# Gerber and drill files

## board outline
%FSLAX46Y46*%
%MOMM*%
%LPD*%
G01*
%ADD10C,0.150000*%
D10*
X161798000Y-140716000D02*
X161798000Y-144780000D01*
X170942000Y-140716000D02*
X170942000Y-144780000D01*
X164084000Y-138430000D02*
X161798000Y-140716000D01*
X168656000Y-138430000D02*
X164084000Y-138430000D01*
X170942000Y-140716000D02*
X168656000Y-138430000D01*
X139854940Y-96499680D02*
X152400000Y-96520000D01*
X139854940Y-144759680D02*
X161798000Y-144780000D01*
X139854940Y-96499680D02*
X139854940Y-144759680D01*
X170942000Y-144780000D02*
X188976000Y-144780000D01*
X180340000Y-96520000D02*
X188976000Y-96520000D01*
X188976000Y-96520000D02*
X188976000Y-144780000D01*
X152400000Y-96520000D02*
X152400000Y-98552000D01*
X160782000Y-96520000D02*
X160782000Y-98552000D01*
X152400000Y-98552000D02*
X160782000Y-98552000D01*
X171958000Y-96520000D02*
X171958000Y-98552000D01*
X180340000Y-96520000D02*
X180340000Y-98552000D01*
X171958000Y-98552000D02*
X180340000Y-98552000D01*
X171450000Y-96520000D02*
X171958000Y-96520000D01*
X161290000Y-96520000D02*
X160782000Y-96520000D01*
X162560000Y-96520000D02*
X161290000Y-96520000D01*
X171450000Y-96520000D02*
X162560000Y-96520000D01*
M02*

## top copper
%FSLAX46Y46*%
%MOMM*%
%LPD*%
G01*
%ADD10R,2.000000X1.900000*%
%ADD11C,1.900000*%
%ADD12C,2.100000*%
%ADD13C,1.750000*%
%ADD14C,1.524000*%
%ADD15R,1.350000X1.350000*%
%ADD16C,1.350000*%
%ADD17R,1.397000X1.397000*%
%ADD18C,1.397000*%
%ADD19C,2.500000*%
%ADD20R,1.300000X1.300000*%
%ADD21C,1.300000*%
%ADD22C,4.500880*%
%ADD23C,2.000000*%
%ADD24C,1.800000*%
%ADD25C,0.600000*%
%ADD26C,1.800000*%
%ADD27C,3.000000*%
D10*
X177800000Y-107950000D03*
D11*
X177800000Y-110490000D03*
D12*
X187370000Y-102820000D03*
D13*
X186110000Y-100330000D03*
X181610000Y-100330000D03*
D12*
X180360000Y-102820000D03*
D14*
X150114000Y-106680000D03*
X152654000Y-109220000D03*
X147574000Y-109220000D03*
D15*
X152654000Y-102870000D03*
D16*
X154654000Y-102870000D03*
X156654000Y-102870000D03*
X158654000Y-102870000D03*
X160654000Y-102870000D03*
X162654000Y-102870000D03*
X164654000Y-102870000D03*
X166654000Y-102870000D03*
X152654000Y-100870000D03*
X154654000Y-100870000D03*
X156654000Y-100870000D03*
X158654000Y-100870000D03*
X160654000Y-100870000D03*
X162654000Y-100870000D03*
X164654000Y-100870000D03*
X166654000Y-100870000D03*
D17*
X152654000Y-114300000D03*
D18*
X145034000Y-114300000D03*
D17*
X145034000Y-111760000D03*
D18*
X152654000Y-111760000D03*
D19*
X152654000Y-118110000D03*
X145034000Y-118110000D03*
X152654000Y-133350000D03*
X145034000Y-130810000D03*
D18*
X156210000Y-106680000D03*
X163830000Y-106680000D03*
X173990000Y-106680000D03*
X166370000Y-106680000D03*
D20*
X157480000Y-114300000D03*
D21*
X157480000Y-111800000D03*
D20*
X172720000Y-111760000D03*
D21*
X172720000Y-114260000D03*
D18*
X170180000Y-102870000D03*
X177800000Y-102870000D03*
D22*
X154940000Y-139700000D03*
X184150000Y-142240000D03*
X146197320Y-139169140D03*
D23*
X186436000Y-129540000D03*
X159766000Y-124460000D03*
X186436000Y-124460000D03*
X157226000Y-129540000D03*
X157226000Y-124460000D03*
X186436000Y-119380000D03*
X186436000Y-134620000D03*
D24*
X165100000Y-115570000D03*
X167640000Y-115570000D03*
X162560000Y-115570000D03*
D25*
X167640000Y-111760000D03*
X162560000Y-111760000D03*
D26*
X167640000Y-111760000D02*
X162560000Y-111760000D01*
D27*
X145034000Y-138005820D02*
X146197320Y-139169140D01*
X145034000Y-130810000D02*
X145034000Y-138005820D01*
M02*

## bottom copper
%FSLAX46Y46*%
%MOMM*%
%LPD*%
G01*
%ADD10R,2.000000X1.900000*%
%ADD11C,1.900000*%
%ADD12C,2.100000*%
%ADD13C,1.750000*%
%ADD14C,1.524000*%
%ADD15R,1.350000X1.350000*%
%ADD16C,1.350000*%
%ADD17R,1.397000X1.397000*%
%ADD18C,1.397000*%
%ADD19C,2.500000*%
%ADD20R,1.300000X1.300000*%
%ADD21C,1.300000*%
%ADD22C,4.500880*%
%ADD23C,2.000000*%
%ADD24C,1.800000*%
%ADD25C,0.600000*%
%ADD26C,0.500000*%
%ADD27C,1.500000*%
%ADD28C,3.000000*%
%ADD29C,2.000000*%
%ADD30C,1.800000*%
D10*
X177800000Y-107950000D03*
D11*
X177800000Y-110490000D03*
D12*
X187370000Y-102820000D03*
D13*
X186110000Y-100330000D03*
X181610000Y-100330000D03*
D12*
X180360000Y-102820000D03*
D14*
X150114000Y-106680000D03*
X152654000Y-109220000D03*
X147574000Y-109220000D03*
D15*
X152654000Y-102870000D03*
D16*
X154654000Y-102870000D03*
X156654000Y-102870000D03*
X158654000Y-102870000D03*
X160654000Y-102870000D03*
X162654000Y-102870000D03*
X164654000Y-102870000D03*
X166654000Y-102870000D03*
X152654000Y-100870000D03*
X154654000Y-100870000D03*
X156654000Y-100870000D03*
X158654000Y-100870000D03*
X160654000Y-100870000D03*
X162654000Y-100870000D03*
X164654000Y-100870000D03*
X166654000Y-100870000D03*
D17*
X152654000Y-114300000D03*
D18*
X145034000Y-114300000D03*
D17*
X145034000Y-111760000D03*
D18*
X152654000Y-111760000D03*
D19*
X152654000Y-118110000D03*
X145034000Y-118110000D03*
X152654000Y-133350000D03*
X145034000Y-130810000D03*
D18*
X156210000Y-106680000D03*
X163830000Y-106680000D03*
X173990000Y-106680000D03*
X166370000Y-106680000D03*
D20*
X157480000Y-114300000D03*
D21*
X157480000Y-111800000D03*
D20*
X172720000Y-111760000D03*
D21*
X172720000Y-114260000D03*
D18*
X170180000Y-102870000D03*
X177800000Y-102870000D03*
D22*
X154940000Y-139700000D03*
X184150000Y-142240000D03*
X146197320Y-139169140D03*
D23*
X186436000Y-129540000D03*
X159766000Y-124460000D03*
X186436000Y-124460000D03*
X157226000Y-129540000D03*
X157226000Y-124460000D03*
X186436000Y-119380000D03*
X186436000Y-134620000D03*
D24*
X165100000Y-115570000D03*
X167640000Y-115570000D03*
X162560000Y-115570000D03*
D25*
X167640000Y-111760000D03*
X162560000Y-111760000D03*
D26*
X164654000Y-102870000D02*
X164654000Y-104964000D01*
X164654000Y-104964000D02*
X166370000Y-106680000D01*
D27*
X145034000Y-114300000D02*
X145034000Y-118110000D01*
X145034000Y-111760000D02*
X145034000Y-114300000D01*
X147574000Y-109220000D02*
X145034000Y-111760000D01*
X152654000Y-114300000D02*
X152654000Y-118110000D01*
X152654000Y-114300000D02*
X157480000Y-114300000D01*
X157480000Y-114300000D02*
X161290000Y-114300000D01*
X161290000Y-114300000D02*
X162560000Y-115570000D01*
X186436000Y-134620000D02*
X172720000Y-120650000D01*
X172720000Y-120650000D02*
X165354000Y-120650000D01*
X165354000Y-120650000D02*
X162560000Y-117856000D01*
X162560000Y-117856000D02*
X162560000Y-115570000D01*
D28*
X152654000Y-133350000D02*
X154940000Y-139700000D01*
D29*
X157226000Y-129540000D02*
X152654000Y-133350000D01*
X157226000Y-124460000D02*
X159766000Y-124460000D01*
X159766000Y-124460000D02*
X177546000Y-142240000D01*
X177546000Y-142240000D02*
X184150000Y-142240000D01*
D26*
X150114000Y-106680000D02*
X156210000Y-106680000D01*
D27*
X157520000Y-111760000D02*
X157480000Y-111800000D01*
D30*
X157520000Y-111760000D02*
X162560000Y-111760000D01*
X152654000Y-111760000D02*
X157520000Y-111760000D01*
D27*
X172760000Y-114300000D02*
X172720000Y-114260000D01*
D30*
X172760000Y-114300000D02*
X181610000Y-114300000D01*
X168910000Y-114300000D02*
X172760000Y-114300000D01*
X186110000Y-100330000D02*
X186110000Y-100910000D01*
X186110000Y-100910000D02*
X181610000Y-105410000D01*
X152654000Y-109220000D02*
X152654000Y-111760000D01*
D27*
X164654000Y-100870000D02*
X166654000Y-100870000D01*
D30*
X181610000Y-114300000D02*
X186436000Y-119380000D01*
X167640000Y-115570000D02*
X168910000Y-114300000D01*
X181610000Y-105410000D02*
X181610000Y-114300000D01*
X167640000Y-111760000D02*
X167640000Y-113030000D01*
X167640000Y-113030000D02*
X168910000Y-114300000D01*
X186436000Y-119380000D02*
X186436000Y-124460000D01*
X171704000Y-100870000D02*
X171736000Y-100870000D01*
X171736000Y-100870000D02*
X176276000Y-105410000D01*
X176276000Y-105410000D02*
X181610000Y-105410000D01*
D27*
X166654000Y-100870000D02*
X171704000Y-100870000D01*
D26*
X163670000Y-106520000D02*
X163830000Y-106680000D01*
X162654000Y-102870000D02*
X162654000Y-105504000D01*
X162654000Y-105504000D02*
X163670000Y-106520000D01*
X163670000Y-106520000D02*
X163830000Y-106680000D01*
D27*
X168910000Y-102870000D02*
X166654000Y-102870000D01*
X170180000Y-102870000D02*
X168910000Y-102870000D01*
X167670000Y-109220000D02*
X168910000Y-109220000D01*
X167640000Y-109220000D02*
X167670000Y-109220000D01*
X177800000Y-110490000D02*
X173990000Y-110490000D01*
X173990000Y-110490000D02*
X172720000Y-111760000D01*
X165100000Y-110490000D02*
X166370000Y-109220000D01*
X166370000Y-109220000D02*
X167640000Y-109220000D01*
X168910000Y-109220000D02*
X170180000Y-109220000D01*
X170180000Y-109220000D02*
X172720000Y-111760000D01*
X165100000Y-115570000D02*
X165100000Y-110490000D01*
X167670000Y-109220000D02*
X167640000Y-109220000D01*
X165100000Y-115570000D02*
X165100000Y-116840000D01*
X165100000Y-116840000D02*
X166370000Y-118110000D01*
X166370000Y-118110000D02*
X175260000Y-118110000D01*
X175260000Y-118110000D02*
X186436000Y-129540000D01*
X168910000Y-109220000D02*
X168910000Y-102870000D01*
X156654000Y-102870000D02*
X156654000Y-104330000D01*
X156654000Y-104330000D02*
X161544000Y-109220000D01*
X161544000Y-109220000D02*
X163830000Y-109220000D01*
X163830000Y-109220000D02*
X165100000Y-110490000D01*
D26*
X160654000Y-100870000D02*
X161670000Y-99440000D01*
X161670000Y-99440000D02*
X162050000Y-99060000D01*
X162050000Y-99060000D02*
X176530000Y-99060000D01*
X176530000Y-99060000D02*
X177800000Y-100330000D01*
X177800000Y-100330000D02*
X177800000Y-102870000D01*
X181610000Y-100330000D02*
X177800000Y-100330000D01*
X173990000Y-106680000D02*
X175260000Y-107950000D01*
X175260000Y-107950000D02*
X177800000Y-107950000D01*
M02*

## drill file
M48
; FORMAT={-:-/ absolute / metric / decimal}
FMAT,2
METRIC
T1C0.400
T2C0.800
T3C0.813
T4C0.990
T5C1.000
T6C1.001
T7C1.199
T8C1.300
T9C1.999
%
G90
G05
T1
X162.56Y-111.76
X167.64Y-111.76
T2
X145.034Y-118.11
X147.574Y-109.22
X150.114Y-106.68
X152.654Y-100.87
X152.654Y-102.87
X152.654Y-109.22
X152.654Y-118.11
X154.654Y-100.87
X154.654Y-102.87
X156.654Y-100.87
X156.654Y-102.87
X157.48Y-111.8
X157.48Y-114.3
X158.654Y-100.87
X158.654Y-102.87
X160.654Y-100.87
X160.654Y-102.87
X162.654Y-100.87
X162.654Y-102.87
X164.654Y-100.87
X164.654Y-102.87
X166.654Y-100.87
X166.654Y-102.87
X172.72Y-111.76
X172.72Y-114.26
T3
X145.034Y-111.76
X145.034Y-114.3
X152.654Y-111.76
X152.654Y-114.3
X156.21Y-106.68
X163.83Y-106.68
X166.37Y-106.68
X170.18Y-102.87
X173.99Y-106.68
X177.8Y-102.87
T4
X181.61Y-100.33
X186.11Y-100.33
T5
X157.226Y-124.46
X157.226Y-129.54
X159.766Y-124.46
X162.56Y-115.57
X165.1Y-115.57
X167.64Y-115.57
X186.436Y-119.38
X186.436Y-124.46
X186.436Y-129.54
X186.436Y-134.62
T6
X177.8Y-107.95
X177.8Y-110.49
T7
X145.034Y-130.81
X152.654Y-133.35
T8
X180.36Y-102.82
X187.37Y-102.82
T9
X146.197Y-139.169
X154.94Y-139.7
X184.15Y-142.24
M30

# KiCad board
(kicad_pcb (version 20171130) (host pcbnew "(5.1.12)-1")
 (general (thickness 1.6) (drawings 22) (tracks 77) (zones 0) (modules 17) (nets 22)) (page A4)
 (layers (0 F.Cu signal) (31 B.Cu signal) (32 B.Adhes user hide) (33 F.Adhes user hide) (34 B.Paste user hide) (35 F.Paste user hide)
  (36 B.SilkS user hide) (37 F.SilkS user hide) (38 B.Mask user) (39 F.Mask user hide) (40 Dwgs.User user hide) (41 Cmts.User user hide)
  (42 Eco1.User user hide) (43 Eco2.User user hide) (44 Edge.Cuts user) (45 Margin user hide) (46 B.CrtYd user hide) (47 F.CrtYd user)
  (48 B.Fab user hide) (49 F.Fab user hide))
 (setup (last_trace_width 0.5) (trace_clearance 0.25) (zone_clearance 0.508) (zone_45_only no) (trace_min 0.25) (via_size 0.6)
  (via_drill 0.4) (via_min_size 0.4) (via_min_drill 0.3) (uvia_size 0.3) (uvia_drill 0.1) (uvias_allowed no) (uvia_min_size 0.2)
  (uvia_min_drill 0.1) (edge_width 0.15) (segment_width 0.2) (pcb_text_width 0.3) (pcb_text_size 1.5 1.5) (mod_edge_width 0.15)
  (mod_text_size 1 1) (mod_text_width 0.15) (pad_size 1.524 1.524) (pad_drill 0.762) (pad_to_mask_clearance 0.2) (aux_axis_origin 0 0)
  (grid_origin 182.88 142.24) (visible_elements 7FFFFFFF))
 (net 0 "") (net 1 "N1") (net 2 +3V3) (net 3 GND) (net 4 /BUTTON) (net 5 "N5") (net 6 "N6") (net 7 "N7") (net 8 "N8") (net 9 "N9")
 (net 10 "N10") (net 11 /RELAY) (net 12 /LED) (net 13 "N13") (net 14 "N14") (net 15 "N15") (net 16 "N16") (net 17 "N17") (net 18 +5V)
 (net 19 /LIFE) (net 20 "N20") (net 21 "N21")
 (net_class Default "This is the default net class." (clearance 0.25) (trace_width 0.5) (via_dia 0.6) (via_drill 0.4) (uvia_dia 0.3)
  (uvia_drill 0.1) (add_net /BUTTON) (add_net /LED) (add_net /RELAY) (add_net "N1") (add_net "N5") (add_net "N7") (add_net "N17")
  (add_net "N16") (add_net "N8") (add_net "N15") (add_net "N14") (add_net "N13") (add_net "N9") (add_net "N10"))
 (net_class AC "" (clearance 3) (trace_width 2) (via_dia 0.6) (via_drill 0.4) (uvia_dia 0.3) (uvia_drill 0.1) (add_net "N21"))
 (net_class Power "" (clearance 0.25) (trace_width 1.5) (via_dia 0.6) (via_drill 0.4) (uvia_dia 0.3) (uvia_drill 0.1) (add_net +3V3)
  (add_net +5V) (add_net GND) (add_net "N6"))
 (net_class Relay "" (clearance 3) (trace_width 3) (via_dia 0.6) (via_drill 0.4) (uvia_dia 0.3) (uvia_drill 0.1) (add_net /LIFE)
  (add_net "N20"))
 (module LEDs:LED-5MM (layer F.Cu) (at 177.8 107.95 270)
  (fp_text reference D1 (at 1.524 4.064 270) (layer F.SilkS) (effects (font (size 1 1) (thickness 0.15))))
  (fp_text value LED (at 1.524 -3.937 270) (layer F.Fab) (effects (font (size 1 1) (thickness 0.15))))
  (pad 1 thru_hole rect (at 0 0) (size 2 1.9) (drill 1.00076) (layers *.Cu *.Mask F.SilkS) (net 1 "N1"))
  (pad 2 thru_hole circle (at 2.54 0 270) (size 1.9 1.9) (drill 1.00076) (layers *.Cu *.Mask F.SilkS) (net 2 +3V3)))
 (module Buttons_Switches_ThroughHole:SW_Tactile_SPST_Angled (layer F.Cu) (at 181.61 100.33)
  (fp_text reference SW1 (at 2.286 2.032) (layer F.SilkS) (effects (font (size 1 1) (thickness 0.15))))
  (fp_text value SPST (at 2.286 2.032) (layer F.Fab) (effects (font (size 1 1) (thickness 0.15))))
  (pad "" thru_hole circle (at 5.76 2.49) (size 2.1 2.1) (drill 1.3) (layers *.Cu *.Mask F.SilkS))
  (pad 2 thru_hole circle (at 4.5 0) (size 1.75 1.75) (drill 0.99) (layers *.Cu *.Mask F.SilkS) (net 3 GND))
  (pad 1 thru_hole circle (at 0 0) (size 1.75 1.75) (drill 0.99) (layers *.Cu *.Mask F.SilkS) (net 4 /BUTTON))
  (pad "" thru_hole circle (at -1.25 2.49) (size 2.1 2.1) (drill 1.3) (layers *.Cu *.Mask F.SilkS)))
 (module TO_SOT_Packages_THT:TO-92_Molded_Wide (layer F.Cu) (at 147.574 109.22)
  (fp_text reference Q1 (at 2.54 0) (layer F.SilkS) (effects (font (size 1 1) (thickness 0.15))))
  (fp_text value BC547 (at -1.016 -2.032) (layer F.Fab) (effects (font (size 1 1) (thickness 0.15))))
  (pad 2 thru_hole circle (at 2.54 -2.54 90) (size 1.524 1.524) (drill 0.8) (layers *.Cu *.Mask F.SilkS) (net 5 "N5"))
  (pad 3 thru_hole circle (at 5.08 0 90) (size 1.524 1.524) (drill 0.8) (layers *.Cu *.Mask F.SilkS) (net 3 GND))
  (pad 1 thru_hole circle (at 0 0 90) (size 1.524 1.524) (drill 0.8) (layers *.Cu *.Mask F.SilkS) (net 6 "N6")))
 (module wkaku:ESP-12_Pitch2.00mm (layer F.Cu) (at 152.654 102.87 90)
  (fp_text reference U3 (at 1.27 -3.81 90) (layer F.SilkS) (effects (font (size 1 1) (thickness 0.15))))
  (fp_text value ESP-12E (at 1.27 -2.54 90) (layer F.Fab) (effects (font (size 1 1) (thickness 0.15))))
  (pad 1 thru_hole rect (at 0 0 90) (size 1.35 1.35) (drill 0.8) (layers *.Cu *.Mask) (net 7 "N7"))
  (pad 2 thru_hole circle (at 0 2 90) (size 1.35 1.35) (drill 0.8) (layers *.Cu *.Mask) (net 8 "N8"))
  (pad 3 thru_hole circle (at 0 4 90) (size 1.35 1.35) (drill 0.8) (layers *.Cu *.Mask) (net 2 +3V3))
  (pad 4 thru_hole circle (at 0 6 90) (size 1.35 1.35) (drill 0.8) (layers *.Cu *.Mask) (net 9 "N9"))
  (pad 5 thru_hole circle (at 0 8 90) (size 1.35 1.35) (drill 0.8) (layers *.Cu *.Mask) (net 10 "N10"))
  (pad 6 thru_hole circle (at 0 10 90) (size 1.35 1.35) (drill 0.8) (layers *.Cu *.Mask) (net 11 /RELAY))
  (pad 7 thru_hole circle (at 0 12 90) (size 1.35 1.35) (drill 0.8) (layers *.Cu *.Mask) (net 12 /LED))
  (pad 8 thru_hole circle (at 0 14 90) (size 1.35 1.35) (drill 0.8) (layers *.Cu *.Mask) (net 2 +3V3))
  (pad 22 thru_hole circle (at 2 0 90) (size 1.35 1.35) (drill 0.8) (layers *.Cu *.Mask) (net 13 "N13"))
  (pad 21 thru_hole circle (at 2 2 90) (size 1.35 1.35) (drill 0.8) (layers *.Cu *.Mask) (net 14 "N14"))
  (pad 20 thru_hole circle (at 2 4 90) (size 1.35 1.35) (drill 0.8) (layers *.Cu *.Mask) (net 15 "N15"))
  (pad 19 thru_hole circle (at 2 6 90) (size 1.35 1.35) (drill 0.8) (layers *.Cu *.Mask) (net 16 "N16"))
  (pad 18 thru_hole circle (at 2 8 90) (size 1.35 1.35) (drill 0.8) (layers *.Cu *.Mask) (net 4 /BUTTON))
  (pad 17 thru_hole circle (at 2 10 90) (size 1.35 1.35) (drill 0.8) (layers *.Cu *.Mask) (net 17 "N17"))
  (pad 16 thru_hole circle (at 2 12 90) (size 1.35 1.35) (drill 0.8) (layers *.Cu *.Mask) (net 3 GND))
  (pad 15 thru_hole circle (at 2 14 90) (size 1.35 1.35) (drill 0.8) (layers *.Cu *.Mask) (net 3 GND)))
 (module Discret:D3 (layer F.Cu) (at 148.844 114.3)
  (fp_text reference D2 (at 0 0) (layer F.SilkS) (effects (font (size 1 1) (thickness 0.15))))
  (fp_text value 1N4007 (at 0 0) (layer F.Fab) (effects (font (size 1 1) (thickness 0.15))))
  (pad 1 thru_hole rect (at 3.81 0) (size 1.397 1.397) (drill 0.8128) (layers *.Cu *.Mask F.SilkS) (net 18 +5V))
  (pad 2 thru_hole circle (at -3.81 0) (size 1.397 1.397) (drill 0.8128) (layers *.Cu *.Mask F.SilkS) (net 6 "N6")))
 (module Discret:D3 (layer F.Cu) (at 148.844 111.76 180)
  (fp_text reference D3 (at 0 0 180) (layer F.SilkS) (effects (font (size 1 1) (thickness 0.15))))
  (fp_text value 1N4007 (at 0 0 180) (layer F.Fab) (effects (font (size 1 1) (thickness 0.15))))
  (pad 1 thru_hole rect (at 3.81 0 180) (size 1.397 1.397) (drill 0.8128) (layers *.Cu *.Mask F.SilkS) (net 6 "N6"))
  (pad 2 thru_hole circle (at -3.81 0 180) (size 1.397 1.397) (drill 0.8128) (layers *.Cu *.Mask F.SilkS) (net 3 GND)))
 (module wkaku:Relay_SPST (layer F.Cu) (at 145.034 118.11 270)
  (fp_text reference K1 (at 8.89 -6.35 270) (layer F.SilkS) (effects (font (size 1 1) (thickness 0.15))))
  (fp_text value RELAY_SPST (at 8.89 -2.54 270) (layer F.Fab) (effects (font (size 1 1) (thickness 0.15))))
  (pad A1 thru_hole circle (at 0 -7.62 270) (size 2.5 2.5) (drill 0.8) (layers *.Cu *.Mask F.SilkS) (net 18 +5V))
  (pad A2 thru_hole circle (at 0 0 270) (size 2.5 2.5) (drill 0.8) (layers *.Cu *.Mask F.SilkS) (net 6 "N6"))
  (pad 7 thru_hole circle (at 15.24 -7.62 270) (size 2.5 2.5) (drill 1.19888) (layers *.Cu *.Mask F.SilkS) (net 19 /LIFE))
  (pad 5 thru_hole circle (at 12.7 0 270) (size 2.5 2.5) (drill 1.19888) (layers *.Cu *.Mask F.SilkS) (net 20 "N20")))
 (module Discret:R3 (layer F.Cu) (at 160.02 106.68)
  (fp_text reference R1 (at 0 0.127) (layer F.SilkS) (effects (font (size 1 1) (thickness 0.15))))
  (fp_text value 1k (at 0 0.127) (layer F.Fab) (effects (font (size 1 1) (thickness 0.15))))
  (pad 1 thru_hole circle (at -3.81 0) (size 1.397 1.397) (drill 0.8128) (layers *.Cu *.Mask F.SilkS) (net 5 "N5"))
  (pad 2 thru_hole circle (at 3.81 0) (size 1.397 1.397) (drill 0.8128) (layers *.Cu *.Mask F.SilkS) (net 11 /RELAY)))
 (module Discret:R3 (layer F.Cu) (at 170.18 106.68 180)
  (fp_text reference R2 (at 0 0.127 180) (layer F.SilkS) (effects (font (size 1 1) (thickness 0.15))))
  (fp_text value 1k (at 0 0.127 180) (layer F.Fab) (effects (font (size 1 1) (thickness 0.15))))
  (pad 1 thru_hole circle (at -3.81 0 180) (size 1.397 1.397) (drill 0.8128) (layers *.Cu *.Mask F.SilkS) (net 1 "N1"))
  (pad 2 thru_hole circle (at 3.81 0 180) (size 1.397 1.397) (drill 0.8128) (layers *.Cu *.Mask F.SilkS) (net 12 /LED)))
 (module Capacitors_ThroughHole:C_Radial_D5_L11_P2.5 (layer F.Cu) (at 157.48 114.3 90)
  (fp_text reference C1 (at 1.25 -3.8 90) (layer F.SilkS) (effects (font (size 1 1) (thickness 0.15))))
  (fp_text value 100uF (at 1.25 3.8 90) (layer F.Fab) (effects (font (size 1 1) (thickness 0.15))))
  (pad 1 thru_hole rect (at 0 0 90) (size 1.3 1.3) (drill 0.8) (layers *.Cu *.Mask F.SilkS) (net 18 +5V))
  (pad 2 thru_hole circle (at 2.5 0 90) (size 1.3 1.3) (drill 0.8) (layers *.Cu *.Mask F.SilkS) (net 3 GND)))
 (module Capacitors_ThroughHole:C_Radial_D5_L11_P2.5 (layer F.Cu) (at 172.72 111.76 270)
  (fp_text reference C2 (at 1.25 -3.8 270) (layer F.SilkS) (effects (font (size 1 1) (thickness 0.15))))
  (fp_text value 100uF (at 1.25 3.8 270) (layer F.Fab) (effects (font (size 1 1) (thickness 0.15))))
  (pad 1 thru_hole rect (at 0 0 270) (size 1.3 1.3) (drill 0.8) (layers *.Cu *.Mask F.SilkS) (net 2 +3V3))
  (pad 2 thru_hole circle (at 2.5 0 270) (size 1.3 1.3) (drill 0.8) (layers *.Cu *.Mask F.SilkS) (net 3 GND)))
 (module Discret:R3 (layer F.Cu) (at 173.99 102.87)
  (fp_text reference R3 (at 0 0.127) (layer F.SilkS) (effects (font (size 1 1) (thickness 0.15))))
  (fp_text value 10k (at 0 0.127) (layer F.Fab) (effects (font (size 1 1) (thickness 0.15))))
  (pad 1 thru_hole circle (at -3.81 0) (size 1.397 1.397) (drill 0.8128) (layers *.Cu *.Mask F.SilkS) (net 2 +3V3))
  (pad 2 thru_hole circle (at 3.81 0) (size 1.397 1.397) (drill 0.8128) (layers *.Cu *.Mask F.SilkS) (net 4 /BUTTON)))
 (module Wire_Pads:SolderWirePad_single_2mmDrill (layer F.Cu) (at 154.94 139.7)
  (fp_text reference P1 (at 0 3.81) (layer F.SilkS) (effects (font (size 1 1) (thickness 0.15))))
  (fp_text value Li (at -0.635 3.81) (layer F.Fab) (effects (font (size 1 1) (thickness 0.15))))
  (pad 1 thru_hole circle (at 0 0) (size 4.50088 4.50088) (drill 1.99898) (layers *.Cu *.Mask F.SilkS) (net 19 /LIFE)))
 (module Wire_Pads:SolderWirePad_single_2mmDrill (layer F.Cu) (at 184.15 142.24)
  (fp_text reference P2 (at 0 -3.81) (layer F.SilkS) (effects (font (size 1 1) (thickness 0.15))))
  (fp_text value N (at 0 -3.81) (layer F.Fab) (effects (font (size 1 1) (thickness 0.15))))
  (pad 1 thru_hole circle (at 0 0) (size 4.50088 4.50088) (drill 1.99898) (layers *.Cu *.Mask F.SilkS) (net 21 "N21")))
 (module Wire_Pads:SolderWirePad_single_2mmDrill (layer F.Cu) (at 146.19732 139.16914)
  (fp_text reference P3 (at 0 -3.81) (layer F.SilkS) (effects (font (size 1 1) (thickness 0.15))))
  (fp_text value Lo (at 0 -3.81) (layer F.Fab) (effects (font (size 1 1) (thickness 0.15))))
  (pad 1 thru_hole circle (at 0 0) (size 4.50088 4.50088) (drill 1.99898) (layers *.Cu *.Mask F.SilkS) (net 20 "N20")))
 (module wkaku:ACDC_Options (layer F.Cu) (at 157.226 129.54)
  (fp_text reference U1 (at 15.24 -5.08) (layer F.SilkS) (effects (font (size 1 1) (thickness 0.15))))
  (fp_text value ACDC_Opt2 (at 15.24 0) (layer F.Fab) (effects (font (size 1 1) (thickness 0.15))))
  (pad 4 thru_hole circle (at 29.21 0) (size 2 2) (drill 1) (layers *.Cu *.Mask F.SilkS) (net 2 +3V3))
  (pad 7 thru_hole circle (at 2.54 -5.08) (size 2 2) (drill 1) (layers *.Cu *.Mask F.SilkS) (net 21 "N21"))
  (pad 6 thru_hole circle (at 29.21 -5.08) (size 2 2) (drill 1) (layers *.Cu *.Mask F.SilkS) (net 3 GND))
  (pad 1 thru_hole circle (at 0 0) (size 2 2) (drill 1) (layers *.Cu *.Mask F.SilkS) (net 19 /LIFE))
  (pad 2 thru_hole circle (at 0 -5.08) (size 2 2) (drill 1) (layers *.Cu *.Mask F.SilkS) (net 21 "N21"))
  (pad 5 thru_hole circle (at 29.21 -10.16) (size 2 2) (drill 1) (layers *.Cu *.Mask F.SilkS) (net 3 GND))
  (pad 3 thru_hole circle (at 29.21 5.08) (size 2 2) (drill 1) (layers *.Cu *.Mask F.SilkS) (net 18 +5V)))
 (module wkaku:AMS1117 (layer F.Cu) (at 165.1 115.57)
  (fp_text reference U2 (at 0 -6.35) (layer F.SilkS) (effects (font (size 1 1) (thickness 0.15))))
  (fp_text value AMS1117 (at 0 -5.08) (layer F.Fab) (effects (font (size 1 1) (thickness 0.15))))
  (pad 2 thru_hole circle (at 0 0) (size 1.8 1.8) (drill 1) (layers *.Cu *.Mask F.SilkS) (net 2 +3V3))
  (pad 1 thru_hole circle (at 2.54 0) (size 1.8 1.8) (drill 1) (layers *.Cu *.Mask F.SilkS) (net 3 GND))
  (pad 3 thru_hole circle (at -2.54 0) (size 1.8 1.8) (drill 1) (layers *.Cu *.Mask F.SilkS) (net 18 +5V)))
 (gr_line (start 161.798 140.716) (end 161.798 144.78) (angle 90) (layer Edge.Cuts) (width 0.15))
 (gr_line (start 170.942 140.716) (end 170.942 144.78) (angle 90) (layer Edge.Cuts) (width 0.15))
 (gr_line (start 164.084 138.43) (end 161.798 140.716) (angle 90) (layer Edge.Cuts) (width 0.15))
 (gr_line (start 168.656 138.43) (end 164.084 138.43) (angle 90) (layer Edge.Cuts) (width 0.15))
 (gr_line (start 170.942 140.716) (end 168.656 138.43) (angle 90) (layer Edge.Cuts) (width 0.15))
 (gr_line (start 139.85494 96.49968) (end 152.4 96.52) (angle 90) (layer Edge.Cuts) (width 0.15))
 (gr_line (start 139.85494 144.75968) (end 161.798 144.78) (angle 90) (layer Edge.Cuts) (width 0.15))
 (gr_line (start 139.85494 96.49968) (end 139.85494 144.75968) (angle 90) (layer Edge.Cuts) (width 0.15))
 (gr_line (start 170.942 144.78) (end 188.976 144.78) (angle 90) (layer Edge.Cuts) (width 0.15))
 (gr_line (start 180.34 96.52) (end 188.976 96.52) (angle 90) (layer Edge.Cuts) (width 0.15))
 (gr_line (start 188.976 96.52) (end 188.976 144.78) (angle 90) (layer Edge.Cuts) (width 0.15))
 (gr_line (start 152.4 96.52) (end 152.4 98.552) (angle 90) (layer Edge.Cuts) (width 0.15))
 (gr_line (start 160.782 96.52) (end 160.782 98.552) (angle 90) (layer Edge.Cuts) (width 0.15))
 (gr_line (start 152.4 98.552) (end 160.782 98.552) (angle 90) (layer Edge.Cuts) (width 0.15))
 (gr_line (start 171.958 96.52) (end 171.958 98.552) (angle 90) (layer Edge.Cuts) (width 0.15))
 (gr_line (start 180.34 96.52) (end 180.34 98.552) (angle 90) (layer Edge.Cuts) (width 0.15))
 (gr_line (start 171.958 98.552) (end 180.34 98.552) (angle 90) (layer Edge.Cuts) (width 0.15))
 (gr_line (start 171.45 96.52) (end 171.958 96.52) (angle 90) (layer Edge.Cuts) (width 0.15))
 (gr_line (start 161.29 96.52) (end 160.782 96.52) (angle 90) (layer Edge.Cuts) (width 0.15))
 (gr_line (start 162.56 96.52) (end 161.29 96.52) (angle 90) (layer Edge.Cuts) (width 0.15))
 (gr_line (start 171.45 96.52) (end 162.56 96.52) (angle 90) (layer Edge.Cuts) (width 0.15))
 (segment (start 164.654 102.87) (end 164.654 104.964) (width 0.5) (layer B.Cu) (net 12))
 (segment (start 164.654 104.964) (end 166.37 106.68) (width 0.5) (layer B.Cu) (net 12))
 (segment (start 145.034 114.3) (end 145.034 118.11) (width 1.5) (layer B.Cu) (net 6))
 (segment (start 145.034 111.76) (end 145.034 114.3) (width 1.5) (layer B.Cu) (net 6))
 (segment (start 147.574 109.22) (end 145.034 111.76) (width 1.5) (layer B.Cu) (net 6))
 (segment (start 152.654 114.3) (end 152.654 118.11) (width 1.5) (layer B.Cu) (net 18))
 (segment (start 152.654 114.3) (end 157.48 114.3) (width 1.5) (layer B.Cu) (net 18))
 (segment (start 157.48 114.3) (end 161.29 114.3) (width 1.5) (layer B.Cu) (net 18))
 (segment (start 161.29 114.3) (end 162.56 115.57) (width 1.5) (layer B.Cu) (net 18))
 (segment (start 186.436 134.62) (end 172.72 120.65) (width 1.5) (layer B.Cu) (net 18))
 (segment (start 172.72 120.65) (end 165.354 120.65) (width 1.5) (layer B.Cu) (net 18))
 (segment (start 165.354 120.65) (end 162.56 117.856) (width 1.5) (layer B.Cu) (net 18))
 (segment (start 162.56 117.856) (end 162.56 115.57) (width 1.5) (layer B.Cu) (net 18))
 (segment (start 152.654 133.35) (end 154.94 139.7) (width 3) (layer B.Cu) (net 19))
 (segment (start 157.226 129.54) (end 152.654 133.35) (width 2) (layer B.Cu) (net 19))
 (segment (start 157.226 124.46) (end 159.766 124.46) (width 2) (layer B.Cu) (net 21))
 (segment (start 159.766 124.46) (end 177.546 142.24) (width 2) (layer B.Cu) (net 21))
 (segment (start 177.546 142.24) (end 184.15 142.24) (width 2) (layer B.Cu) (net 21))
 (segment (start 150.114 106.68) (end 156.21 106.68) (width 0.5) (layer B.Cu) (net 5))
 (segment (start 157.52 111.76) (end 157.48 111.8) (width 1.5) (layer B.Cu) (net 3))
 (segment (start 157.52 111.76) (end 162.56 111.76) (width 1.8) (layer B.Cu) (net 3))
 (segment (start 152.654 111.76) (end 157.52 111.76) (width 1.8) (layer B.Cu) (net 3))
 (segment (start 172.76 114.3) (end 172.72 114.26) (width 1.5) (layer B.Cu) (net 3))
 (segment (start 172.76 114.3) (end 181.61 114.3) (width 1.8) (layer B.Cu) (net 3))
 (segment (start 168.91 114.3) (end 172.76 114.3) (width 1.8) (layer B.Cu) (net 3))
 (segment (start 186.11 100.33) (end 186.11 100.91) (width 1.8) (layer B.Cu) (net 3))
 (segment (start 186.11 100.91) (end 181.61 105.41) (width 1.8) (layer B.Cu) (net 3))
 (segment (start 152.654 109.22) (end 152.654 111.76) (width 1.8) (layer B.Cu) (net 3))
 (segment (start 164.654 100.87) (end 166.654 100.87) (width 1.5) (layer B.Cu) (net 3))
 (segment (start 181.61 114.3) (end 186.436 119.38) (width 1.8) (layer B.Cu) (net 3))
 (segment (start 167.64 115.57) (end 168.91 114.3) (width 1.8) (layer B.Cu) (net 3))
 (segment (start 181.61 105.41) (end 181.61 114.3) (width 1.8) (layer B.Cu) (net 3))
 (segment (start 167.64 111.76) (end 162.56 111.76) (width 1.8) (layer F.Cu) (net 3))
 (segment (start 167.64 111.76) (end 167.64 113.03) (width 1.8) (layer B.Cu) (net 3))
 (segment (start 167.64 113.03) (end 168.91 114.3) (width 1.8) (layer B.Cu) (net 3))
 (segment (start 186.436 119.38) (end 186.436 124.46) (width 1.8) (layer B.Cu) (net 3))
 (segment (start 171.704 100.87) (end 171.736 100.87) (width 1.8) (layer B.Cu) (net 3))
 (segment (start 171.736 100.87) (end 176.276 105.41) (width 1.8) (layer B.Cu) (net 3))
 (segment (start 176.276 105.41) (end 181.61 105.41) (width 1.8) (layer B.Cu) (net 3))
 (segment (start 166.654 100.87) (end 171.704 100.87) (width 1.5) (layer B.Cu) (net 3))
 (via (at 167.64 111.76) (size 0.6) (layers F.Cu B.Cu) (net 3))
 (via (at 162.56 111.76) (size 0.6) (layers F.Cu B.Cu) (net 3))
 (segment (start 163.67 106.52) (end 163.83 106.68) (width 0.5) (layer B.Cu) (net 11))
 (segment (start 162.654 102.87) (end 162.654 105.504) (width 0.5) (layer B.Cu) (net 11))
 (segment (start 162.654 105.504) (end 163.67 106.52) (width 0.5) (layer B.Cu) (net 11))
 (segment (start 163.67 106.52) (end 163.83 106.68) (width 0.5) (layer B.Cu) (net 11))
 (segment (start 168.91 102.87) (end 166.654 102.87) (width 1.5) (layer B.Cu) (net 2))
 (segment (start 170.18 102.87) (end 168.91 102.87) (width 1.5) (layer B.Cu) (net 2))
 (segment (start 167.67 109.22) (end 168.91 109.22) (width 1.5) (layer B.Cu) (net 2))
 (segment (start 167.64 109.22) (end 167.67 109.22) (width 1.5) (layer B.Cu) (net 2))
 (segment (start 177.8 110.49) (end 173.99 110.49) (width 1.5) (layer B.Cu) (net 2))
 (segment (start 173.99 110.49) (end 172.72 111.76) (width 1.5) (layer B.Cu) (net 2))
 (segment (start 165.1 110.49) (end 166.37 109.22) (width 1.5) (layer B.Cu) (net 2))
 (segment (start 166.37 109.22) (end 167.64 109.22) (width 1.5) (layer B.Cu) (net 2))
 (segment (start 168.91 109.22) (end 170.18 109.22) (width 1.5) (layer B.Cu) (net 2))
 (segment (start 170.18 109.22) (end 172.72 111.76) (width 1.5) (layer B.Cu) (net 2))
 (segment (start 165.1 115.57) (end 165.1 110.49) (width 1.5) (layer B.Cu) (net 2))
 (segment (start 167.67 109.22) (end 167.64 109.22) (width 1.5) (layer B.Cu) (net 2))
 (segment (start 165.1 115.57) (end 165.1 116.84) (width 1.5) (layer B.Cu) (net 2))
 (segment (start 165.1 116.84) (end 166.37 118.11) (width 1.5) (layer B.Cu) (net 2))
 (segment (start 166.37 118.11) (end 175.26 118.11) (width 1.5) (layer B.Cu) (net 2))
 (segment (start 175.26 118.11) (end 186.436 129.54) (width 1.5) (layer B.Cu) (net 2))
 (segment (start 168.91 109.22) (end 168.91 102.87) (width 1.5) (layer B.Cu) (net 2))
 (segment (start 156.654 102.87) (end 156.654 104.33) (width 1.5) (layer B.Cu) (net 2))
 (segment (start 156.654 104.33) (end 161.544 109.22) (width 1.5) (layer B.Cu) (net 2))
 (segment (start 161.544 109.22) (end 163.83 109.22) (width 1.5) (layer B.Cu) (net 2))
 (segment (start 163.83 109.22) (end 165.1 110.49) (width 1.5) (layer B.Cu) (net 2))
 (segment (start 160.654 100.87) (end 161.67 99.44) (width 0.5) (layer B.Cu) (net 4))
 (segment (start 161.67 99.44) (end 162.05 99.06) (width 0.5) (layer B.Cu) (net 4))
 (segment (start 162.05 99.06) (end 176.53 99.06) (width 0.5) (layer B.Cu) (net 4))
 (segment (start 176.53 99.06) (end 177.8 100.33) (width 0.5) (layer B.Cu) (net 4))
 (segment (start 177.8 100.33) (end 177.8 102.87) (width 0.5) (layer B.Cu) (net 4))
 (segment (start 181.61 100.33) (end 177.8 100.33) (width 0.5) (layer B.Cu) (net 4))
 (segment (start 145.034 138.00582) (end 146.19732 139.16914) (width 3) (layer F.Cu) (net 20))
 (segment (start 145.034 130.81) (end 145.034 138.00582) (width 3) (layer F.Cu) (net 20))
 (segment (start 173.99 106.68) (end 175.26 107.95) (width 0.5) (layer B.Cu) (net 1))
 (segment (start 175.26 107.95) (end 177.8 107.95) (width 0.5) (layer B.Cu) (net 1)))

